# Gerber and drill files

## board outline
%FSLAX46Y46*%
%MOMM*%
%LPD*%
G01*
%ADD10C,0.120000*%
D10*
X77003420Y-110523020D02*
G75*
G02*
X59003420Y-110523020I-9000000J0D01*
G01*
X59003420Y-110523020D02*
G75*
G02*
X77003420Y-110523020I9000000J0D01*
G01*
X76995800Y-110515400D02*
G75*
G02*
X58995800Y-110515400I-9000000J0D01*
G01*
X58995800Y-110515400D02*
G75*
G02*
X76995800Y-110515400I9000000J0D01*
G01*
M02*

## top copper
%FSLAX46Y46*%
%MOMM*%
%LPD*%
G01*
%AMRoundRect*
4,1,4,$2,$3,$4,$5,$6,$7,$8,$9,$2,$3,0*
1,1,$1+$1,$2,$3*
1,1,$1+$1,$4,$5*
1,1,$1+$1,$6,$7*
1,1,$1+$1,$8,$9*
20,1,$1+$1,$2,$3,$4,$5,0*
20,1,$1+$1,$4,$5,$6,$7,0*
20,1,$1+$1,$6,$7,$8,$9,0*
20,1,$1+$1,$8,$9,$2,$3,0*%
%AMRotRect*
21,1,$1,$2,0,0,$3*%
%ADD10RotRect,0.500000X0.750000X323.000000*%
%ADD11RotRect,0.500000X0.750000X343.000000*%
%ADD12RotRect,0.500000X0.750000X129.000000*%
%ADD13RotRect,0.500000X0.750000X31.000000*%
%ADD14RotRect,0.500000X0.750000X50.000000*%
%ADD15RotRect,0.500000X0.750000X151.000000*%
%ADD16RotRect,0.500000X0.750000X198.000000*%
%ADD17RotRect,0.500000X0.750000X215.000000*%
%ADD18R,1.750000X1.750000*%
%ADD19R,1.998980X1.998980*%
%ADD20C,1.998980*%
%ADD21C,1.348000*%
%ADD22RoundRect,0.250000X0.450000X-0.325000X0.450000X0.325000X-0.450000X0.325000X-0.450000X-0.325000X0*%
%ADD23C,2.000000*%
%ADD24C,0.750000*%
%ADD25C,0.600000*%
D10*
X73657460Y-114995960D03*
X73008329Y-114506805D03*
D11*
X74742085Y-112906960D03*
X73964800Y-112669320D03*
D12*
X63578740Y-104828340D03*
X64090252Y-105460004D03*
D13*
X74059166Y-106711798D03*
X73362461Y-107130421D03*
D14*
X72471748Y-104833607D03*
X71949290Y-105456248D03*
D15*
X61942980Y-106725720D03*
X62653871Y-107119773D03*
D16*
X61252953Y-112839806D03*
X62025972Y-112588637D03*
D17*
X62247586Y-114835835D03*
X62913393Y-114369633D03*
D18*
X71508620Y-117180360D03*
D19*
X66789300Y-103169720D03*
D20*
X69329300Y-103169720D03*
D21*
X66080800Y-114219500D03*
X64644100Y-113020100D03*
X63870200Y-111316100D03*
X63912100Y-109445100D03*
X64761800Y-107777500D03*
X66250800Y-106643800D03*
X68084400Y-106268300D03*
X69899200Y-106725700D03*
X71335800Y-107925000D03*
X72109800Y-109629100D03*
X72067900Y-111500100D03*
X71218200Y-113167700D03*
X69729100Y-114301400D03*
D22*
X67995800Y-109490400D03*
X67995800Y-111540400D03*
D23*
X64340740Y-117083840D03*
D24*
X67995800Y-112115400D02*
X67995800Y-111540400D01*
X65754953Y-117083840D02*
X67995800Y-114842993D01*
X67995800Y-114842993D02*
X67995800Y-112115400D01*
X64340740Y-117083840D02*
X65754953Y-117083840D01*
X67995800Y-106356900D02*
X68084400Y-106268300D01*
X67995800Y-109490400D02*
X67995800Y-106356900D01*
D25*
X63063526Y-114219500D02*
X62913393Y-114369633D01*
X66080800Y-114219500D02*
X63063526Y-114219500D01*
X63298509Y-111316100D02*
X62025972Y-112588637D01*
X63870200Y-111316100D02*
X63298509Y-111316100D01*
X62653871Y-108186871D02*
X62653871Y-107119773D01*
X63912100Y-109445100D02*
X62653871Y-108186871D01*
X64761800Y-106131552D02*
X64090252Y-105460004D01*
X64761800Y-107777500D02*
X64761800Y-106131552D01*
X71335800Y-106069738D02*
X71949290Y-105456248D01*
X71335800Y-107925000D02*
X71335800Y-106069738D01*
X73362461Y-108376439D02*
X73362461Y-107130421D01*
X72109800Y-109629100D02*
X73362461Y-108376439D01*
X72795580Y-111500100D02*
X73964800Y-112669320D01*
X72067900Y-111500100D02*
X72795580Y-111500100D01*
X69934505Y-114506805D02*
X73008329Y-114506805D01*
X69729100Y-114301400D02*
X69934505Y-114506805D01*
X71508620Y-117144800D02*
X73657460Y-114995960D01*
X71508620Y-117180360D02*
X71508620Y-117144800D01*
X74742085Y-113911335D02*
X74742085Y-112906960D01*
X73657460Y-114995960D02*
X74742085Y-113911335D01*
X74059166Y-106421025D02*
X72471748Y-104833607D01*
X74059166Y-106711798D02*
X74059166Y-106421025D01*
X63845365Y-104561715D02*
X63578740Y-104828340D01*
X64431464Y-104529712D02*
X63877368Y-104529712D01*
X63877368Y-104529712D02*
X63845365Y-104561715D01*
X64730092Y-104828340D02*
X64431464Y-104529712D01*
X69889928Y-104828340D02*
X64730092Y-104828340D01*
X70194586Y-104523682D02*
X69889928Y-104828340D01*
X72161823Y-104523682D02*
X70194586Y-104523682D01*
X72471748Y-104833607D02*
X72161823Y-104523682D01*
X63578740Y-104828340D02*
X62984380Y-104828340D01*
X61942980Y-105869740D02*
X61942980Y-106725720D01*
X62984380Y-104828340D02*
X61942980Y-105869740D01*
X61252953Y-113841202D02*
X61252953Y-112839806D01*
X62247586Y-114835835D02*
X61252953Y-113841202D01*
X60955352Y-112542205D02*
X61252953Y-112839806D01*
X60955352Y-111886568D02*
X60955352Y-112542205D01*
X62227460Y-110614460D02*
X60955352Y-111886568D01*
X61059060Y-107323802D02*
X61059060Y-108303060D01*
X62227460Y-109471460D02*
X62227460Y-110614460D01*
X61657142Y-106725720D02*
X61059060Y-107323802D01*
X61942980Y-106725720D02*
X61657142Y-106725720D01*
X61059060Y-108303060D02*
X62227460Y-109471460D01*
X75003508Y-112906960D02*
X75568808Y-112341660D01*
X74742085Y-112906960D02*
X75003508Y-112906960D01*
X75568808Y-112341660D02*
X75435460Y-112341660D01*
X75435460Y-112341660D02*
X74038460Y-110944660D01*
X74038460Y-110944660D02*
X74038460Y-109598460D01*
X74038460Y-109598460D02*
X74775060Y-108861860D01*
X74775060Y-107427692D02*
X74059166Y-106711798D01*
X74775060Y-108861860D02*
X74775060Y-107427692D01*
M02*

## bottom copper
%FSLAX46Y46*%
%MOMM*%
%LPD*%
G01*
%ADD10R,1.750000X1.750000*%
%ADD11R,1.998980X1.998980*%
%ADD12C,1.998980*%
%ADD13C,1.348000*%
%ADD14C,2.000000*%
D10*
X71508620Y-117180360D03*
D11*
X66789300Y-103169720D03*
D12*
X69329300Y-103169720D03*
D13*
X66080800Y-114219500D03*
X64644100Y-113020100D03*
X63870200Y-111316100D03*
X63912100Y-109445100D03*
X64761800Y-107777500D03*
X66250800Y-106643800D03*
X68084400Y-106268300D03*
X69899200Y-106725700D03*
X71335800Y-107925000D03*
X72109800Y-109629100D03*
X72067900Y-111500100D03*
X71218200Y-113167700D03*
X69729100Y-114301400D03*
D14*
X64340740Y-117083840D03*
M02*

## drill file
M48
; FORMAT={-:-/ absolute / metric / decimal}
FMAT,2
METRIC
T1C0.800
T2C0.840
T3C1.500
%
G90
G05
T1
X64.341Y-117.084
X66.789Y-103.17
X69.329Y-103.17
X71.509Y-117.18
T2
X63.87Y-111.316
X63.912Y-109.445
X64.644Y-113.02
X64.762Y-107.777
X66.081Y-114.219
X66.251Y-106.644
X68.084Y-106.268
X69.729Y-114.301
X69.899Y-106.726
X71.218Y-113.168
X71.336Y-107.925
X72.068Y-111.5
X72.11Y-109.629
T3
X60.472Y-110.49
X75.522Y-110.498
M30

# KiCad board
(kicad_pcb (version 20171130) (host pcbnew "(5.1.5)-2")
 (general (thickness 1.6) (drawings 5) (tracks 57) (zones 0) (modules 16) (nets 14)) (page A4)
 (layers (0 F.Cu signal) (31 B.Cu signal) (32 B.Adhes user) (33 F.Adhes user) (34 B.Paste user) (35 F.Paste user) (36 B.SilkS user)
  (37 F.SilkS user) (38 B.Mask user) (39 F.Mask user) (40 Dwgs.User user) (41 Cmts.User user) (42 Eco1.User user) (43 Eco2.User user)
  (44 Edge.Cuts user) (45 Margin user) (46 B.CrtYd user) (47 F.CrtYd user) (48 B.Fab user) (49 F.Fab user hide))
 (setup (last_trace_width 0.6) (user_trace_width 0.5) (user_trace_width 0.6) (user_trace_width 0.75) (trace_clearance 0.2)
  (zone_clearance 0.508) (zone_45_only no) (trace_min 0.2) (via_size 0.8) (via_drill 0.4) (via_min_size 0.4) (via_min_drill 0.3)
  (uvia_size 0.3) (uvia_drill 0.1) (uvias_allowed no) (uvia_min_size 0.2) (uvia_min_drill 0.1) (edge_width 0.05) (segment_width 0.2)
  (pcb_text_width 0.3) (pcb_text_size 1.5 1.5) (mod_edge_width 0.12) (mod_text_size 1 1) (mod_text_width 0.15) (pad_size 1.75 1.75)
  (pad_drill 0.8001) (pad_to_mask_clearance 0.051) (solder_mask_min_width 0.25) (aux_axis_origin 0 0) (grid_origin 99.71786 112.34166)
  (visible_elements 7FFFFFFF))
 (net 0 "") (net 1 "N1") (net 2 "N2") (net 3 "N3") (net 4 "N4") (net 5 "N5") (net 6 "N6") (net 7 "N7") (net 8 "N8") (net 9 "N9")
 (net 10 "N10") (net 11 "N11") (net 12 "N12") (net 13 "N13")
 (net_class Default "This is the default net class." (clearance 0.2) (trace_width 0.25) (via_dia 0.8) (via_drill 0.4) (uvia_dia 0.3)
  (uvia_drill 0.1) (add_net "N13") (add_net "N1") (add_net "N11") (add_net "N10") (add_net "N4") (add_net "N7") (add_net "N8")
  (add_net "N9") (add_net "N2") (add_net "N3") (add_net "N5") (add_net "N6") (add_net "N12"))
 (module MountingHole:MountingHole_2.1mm (layer F.Cu) (at 60.47232 110.49)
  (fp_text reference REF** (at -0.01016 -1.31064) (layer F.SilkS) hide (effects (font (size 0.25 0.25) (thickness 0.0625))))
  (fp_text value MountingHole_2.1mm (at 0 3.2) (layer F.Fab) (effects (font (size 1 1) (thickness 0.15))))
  (pad "" np_thru_hole circle (at 0 0) (size 1.5 1.5) (drill 1.5) (layers *.Cu *.Mask)))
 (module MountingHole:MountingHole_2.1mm (layer F.Cu) (at 75.52182 110.49762)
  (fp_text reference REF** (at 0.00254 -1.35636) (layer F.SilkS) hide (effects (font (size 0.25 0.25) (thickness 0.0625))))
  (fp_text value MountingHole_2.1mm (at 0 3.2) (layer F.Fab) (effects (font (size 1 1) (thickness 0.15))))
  (pad "" np_thru_hole circle (at 0 0) (size 1.5 1.5) (drill 1.5) (layers *.Cu *.Mask)))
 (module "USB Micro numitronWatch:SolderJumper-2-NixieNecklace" (layer F.Cu) (at 73.530749 114.868672 323)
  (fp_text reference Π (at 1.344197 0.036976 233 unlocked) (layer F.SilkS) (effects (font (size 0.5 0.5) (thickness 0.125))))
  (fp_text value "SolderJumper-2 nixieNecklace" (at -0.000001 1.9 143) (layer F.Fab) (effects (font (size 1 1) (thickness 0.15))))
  (pad 2 smd rect (at 0.1778 0.0254 323) (size 0.5 0.75) (layers F.Cu F.Mask) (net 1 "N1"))
  (pad 1 smd rect (at -0.635 0.0254 323) (size 0.5 0.75) (layers F.Cu F.Mask) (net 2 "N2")))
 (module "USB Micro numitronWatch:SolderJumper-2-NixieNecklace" (layer F.Cu) (at 74.57948 112.830686 343)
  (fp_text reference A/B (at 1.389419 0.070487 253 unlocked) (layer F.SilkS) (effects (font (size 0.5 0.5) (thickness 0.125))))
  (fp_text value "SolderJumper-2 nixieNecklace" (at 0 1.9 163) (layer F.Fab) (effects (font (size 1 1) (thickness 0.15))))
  (pad 2 smd rect (at 0.1778 0.0254 343) (size 0.5 0.75) (layers F.Cu F.Mask) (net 1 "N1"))
  (pad 1 smd rect (at -0.635 0.0254 343) (size 0.5 0.75) (layers F.Cu F.Mask) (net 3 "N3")))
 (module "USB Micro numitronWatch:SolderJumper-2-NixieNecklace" (layer F.Cu) (at 63.670894 104.982501 129)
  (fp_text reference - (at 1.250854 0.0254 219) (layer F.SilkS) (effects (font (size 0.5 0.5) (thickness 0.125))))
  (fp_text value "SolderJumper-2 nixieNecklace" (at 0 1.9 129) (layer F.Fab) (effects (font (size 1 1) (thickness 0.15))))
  (pad 2 smd rect (at 0.1778 0.0254 129) (size 0.5 0.75) (layers F.Cu F.Mask) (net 1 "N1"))
  (pad 1 smd rect (at -0.635 0.0254 129) (size 0.5 0.75) (layers F.Cu F.Mask) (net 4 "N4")))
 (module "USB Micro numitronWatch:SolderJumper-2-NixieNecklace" (layer F.Cu) (at 73.89368 106.7816 31)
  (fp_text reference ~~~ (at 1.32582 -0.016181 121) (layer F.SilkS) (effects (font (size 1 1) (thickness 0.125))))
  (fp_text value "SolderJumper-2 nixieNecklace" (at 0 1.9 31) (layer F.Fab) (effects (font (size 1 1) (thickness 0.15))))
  (pad 2 smd rect (at 0.1778 0.0254 31) (size 0.5 0.75) (layers F.Cu F.Mask) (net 1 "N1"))
  (pad 1 smd rect (at -0.635 0.0254 31) (size 0.5 0.75) (layers F.Cu F.Mask) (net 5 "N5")))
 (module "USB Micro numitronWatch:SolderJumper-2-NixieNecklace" (layer F.Cu) (at 72.338003 104.953483 50)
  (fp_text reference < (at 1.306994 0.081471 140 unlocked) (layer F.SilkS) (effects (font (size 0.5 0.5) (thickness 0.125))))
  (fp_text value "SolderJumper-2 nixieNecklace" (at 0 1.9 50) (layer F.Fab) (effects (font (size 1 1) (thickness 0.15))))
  (pad 2 smd rect (at 0.1778 0.0254 50) (size 0.5 0.75) (layers F.Cu F.Mask) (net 1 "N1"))
  (pad 1 smd rect (at -0.635 0.0254 50) (size 0.5 0.75) (layers F.Cu F.Mask) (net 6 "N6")))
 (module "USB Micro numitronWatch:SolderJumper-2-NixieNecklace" (layer F.Cu) (at 62.086173 106.834134 151)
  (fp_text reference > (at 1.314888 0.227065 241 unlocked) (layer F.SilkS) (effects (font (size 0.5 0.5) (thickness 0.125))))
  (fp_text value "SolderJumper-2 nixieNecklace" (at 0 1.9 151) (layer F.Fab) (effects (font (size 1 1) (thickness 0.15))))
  (pad 2 smd rect (at 0.1778 0.0254 151) (size 0.5 0.75) (layers F.Cu F.Mask) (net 1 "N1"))
  (pad 1 smd rect (at -0.635 0.0254 151) (size 0.5 0.75) (layers F.Cu F.Mask) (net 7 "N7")))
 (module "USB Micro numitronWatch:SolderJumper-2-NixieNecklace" (layer F.Cu) (at 61.4299 112.80902 198)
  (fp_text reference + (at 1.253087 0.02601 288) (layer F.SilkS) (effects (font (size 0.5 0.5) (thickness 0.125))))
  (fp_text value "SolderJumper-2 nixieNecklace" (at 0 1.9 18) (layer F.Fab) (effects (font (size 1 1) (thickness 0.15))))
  (pad 2 smd rect (at 0.1778 0.0254 198) (size 0.5 0.75) (layers F.Cu F.Mask) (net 1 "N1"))
  (pad 1 smd rect (at -0.635 0.0254 198) (size 0.5 0.75) (layers F.Cu F.Mask) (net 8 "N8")))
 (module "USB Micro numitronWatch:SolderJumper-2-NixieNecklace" (layer F.Cu) (at 62.4078 114.75466 215)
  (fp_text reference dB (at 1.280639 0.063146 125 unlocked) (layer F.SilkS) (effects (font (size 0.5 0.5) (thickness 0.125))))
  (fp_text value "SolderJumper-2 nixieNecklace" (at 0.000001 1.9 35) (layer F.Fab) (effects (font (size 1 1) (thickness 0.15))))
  (pad 2 smd rect (at 0.1778 0.0254 215) (size 0.5 0.75) (layers F.Cu F.Mask) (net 1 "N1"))
  (pad 1 smd rect (at -0.635 0.0254 215) (size 0.5 0.75) (layers F.Cu F.Mask) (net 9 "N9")))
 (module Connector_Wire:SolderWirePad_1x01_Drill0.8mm (layer F.Cu) (at 71.50862 117.18036)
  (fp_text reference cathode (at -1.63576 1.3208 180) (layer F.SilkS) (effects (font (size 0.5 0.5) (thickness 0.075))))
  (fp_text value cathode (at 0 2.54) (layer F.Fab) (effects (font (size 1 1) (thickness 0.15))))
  (pad 1 thru_hole rect (at 0 0) (size 1.75 1.75) (drill 0.8001) (layers *.Cu *.Mask) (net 1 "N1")))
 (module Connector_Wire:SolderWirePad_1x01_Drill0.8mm (layer F.Cu) (at 66.7893 103.16972)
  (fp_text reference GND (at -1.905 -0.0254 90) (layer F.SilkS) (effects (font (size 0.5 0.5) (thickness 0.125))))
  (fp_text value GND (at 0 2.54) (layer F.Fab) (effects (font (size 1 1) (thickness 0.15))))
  (pad 1 thru_hole rect (at 0 0) (size 1.99898 1.99898) (drill 0.8001) (layers *.Cu *.Mask) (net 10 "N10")))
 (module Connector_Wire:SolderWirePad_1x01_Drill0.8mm (layer F.Cu) (at 69.3293 103.16972)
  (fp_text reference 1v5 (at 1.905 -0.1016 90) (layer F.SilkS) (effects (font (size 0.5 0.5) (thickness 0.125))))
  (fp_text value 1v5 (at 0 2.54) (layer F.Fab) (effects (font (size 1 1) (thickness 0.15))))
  (pad 1 thru_hole circle (at 0 0) (size 1.99898 1.99898) (drill 0.8001) (layers *.Cu *.Mask) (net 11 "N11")))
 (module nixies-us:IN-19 (layer F.Cu) (at 67.9958 110.5154)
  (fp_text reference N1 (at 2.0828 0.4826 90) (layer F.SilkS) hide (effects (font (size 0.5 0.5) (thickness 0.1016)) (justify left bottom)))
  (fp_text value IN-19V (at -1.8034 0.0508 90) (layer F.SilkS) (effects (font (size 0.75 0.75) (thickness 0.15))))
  (pad 14 thru_hole circle (at -1.915 3.7041 333) (size 1.348 1.348) (drill 0.84) (layers *.Cu *.Mask) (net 9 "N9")
   (solder_mask_margin 0.1016))
  (pad 13 thru_hole circle (at -3.3517 2.5047 333) (size 1.348 1.348) (drill 0.84) (layers *.Cu *.Mask) (solder_mask_margin 0.1016))
  (pad 12 thru_hole circle (at -4.1256 0.8007 333) (size 1.348 1.348) (drill 0.84) (layers *.Cu *.Mask) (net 8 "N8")
   (solder_mask_margin 0.1016))
  (pad 11 thru_hole circle (at -4.0837 -1.0703 333) (size 1.348 1.348) (drill 0.84) (layers *.Cu *.Mask) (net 7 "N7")
   (solder_mask_margin 0.1016))
  (pad 10 thru_hole circle (at -3.234 -2.7379 333) (size 1.348 1.348) (drill 0.84) (layers *.Cu *.Mask) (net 4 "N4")
   (solder_mask_margin 0.1016))
  (pad 9 thru_hole circle (at -1.745 -3.8716 333) (size 1.348 1.348) (drill 0.84) (layers *.Cu *.Mask) (solder_mask_margin 0.1016))
  (pad 8 thru_hole circle (at 0.0886 -4.2471 333) (size 1.348 1.348) (drill 0.84) (layers *.Cu *.Mask) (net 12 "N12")
   (solder_mask_margin 0.1016))
  (pad 7 thru_hole circle (at 1.9034 -3.7897 333) (size 1.348 1.348) (drill 0.84) (layers *.Cu *.Mask) (solder_mask_margin 0.1016))
  (pad 6 thru_hole circle (at 3.34 -2.5904 333) (size 1.348 1.348) (drill 0.84) (layers *.Cu *.Mask) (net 6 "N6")
   (solder_mask_margin 0.1016))
  (pad 5 thru_hole circle (at 4.114 -0.8863 333) (size 1.348 1.348) (drill 0.84) (layers *.Cu *.Mask) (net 5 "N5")
   (solder_mask_margin 0.1016))
  (pad 4 thru_hole circle (at 4.0721 0.9847 333) (size 1.348 1.348) (drill 0.84) (layers *.Cu *.Mask) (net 3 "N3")
   (solder_mask_margin 0.1016))
  (pad 3 thru_hole circle (at 3.2224 2.6523 333) (size 1.348 1.348) (drill 0.84) (layers *.Cu *.Mask) (solder_mask_margin 0.1016))
  (pad 2 thru_hole circle (at 1.7333 3.786 333) (size 1.348 1.348) (drill 0.84) (layers *.Cu *.Mask) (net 2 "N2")
   (solder_mask_margin 0.1016)))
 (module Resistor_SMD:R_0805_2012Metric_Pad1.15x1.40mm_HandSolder (layer F.Cu) (at 67.9958 110.5154 90)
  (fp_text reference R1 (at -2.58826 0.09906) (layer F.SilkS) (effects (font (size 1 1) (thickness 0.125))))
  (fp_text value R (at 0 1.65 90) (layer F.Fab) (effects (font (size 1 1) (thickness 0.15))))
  (pad 2 smd roundrect (at 1.025 0 90) (size 1.15 1.4) (layers F.Cu F.Paste F.Mask) (roundrect_rratio 0.217391) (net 12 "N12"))
  (pad 1 smd roundrect (at -1.025 0 90) (size 1.15 1.4) (layers F.Cu F.Paste F.Mask) (roundrect_rratio 0.217391) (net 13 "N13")))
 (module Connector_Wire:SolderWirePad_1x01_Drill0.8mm (layer F.Cu) (at 64.34074 117.08384)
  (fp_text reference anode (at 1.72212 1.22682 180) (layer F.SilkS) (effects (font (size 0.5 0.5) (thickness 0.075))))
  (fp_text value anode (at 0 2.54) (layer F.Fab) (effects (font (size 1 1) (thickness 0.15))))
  (pad 1 thru_hole circle (at 0 0) (size 2 2) (drill 0.8001) (layers *.Cu *.Mask) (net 13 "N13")))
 (gr_circle (center 68.00342 110.52302) (end 77.00342 110.52302) (layer Edge.Cuts) (width 0.12))
 (gr_circle (center 67.9958 110.5154) (end 76.9958 110.5154) (layer Edge.Cuts) (width 0.12))
 (segment (start 67.9958 112.1154) (end 67.9958 111.5404) (width 0.75) (layer F.Cu) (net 13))
 (segment (start 65.754953 117.08384) (end 67.9958 114.842993) (width 0.75) (layer F.Cu) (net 13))
 (segment (start 67.9958 114.842993) (end 67.9958 112.1154) (width 0.75) (layer F.Cu) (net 13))
 (segment (start 64.34074 117.08384) (end 65.754953 117.08384) (width 0.75) (layer F.Cu) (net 13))
 (segment (start 67.9958 106.3569) (end 68.0844 106.2683) (width 0.75) (layer F.Cu) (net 12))
 (segment (start 67.9958 109.4904) (end 67.9958 106.3569) (width 0.75) (layer F.Cu) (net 12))
 (segment (start 63.063526 114.2195) (end 62.913393 114.369633) (width 0.6) (layer F.Cu) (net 9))
 (segment (start 66.0808 114.2195) (end 63.063526 114.2195) (width 0.6) (layer F.Cu) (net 9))
 (segment (start 63.298509 111.3161) (end 62.025972 112.588637) (width 0.6) (layer F.Cu) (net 8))
 (segment (start 63.8702 111.3161) (end 63.298509 111.3161) (width 0.6) (layer F.Cu) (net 8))
 (segment (start 62.653871 108.186871) (end 62.653871 107.119773) (width 0.6) (layer F.Cu) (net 7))
 (segment (start 63.9121 109.4451) (end 62.653871 108.186871) (width 0.6) (layer F.Cu) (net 7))
 (segment (start 64.7618 106.131552) (end 64.090252 105.460004) (width 0.6) (layer F.Cu) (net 4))
 (segment (start 64.7618 107.7775) (end 64.7618 106.131552) (width 0.6) (layer F.Cu) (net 4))
 (segment (start 71.3358 106.069738) (end 71.94929 105.456248) (width 0.6) (layer F.Cu) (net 6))
 (segment (start 71.3358 107.925) (end 71.3358 106.069738) (width 0.6) (layer F.Cu) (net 6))
 (segment (start 73.362461 108.376439) (end 73.362461 107.130421) (width 0.6) (layer F.Cu) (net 5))
 (segment (start 72.1098 109.6291) (end 73.362461 108.376439) (width 0.6) (layer F.Cu) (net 5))
 (segment (start 72.79558 111.5001) (end 73.9648 112.66932) (width 0.6) (layer F.Cu) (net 3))
 (segment (start 72.0679 111.5001) (end 72.79558 111.5001) (width 0.6) (layer F.Cu) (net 3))
 (segment (start 69.934505 114.506805) (end 73.008329 114.506805) (width 0.6) (layer F.Cu) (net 2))
 (segment (start 69.7291 114.3014) (end 69.934505 114.506805) (width 0.6) (layer F.Cu) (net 2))
 (segment (start 71.50862 117.1448) (end 73.65746 114.99596) (width 0.6) (layer F.Cu) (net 1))
 (segment (start 71.50862 117.18036) (end 71.50862 117.1448) (width 0.6) (layer F.Cu) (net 1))
 (segment (start 74.742085 113.911335) (end 74.742085 112.90696) (width 0.6) (layer F.Cu) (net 1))
 (segment (start 73.65746 114.99596) (end 74.742085 113.911335) (width 0.6) (layer F.Cu) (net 1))
 (segment (start 74.059166 106.421025) (end 72.471748 104.833607) (width 0.6) (layer F.Cu) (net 1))
 (segment (start 74.059166 106.711798) (end 74.059166 106.421025) (width 0.6) (layer F.Cu) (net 1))
 (segment (start 63.845365 104.561715) (end 63.57874 104.82834) (width 0.6) (layer F.Cu) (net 1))
 (segment (start 64.431464 104.529712) (end 63.877368 104.529712) (width 0.6) (layer F.Cu) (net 1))
 (segment (start 63.877368 104.529712) (end 63.845365 104.561715) (width 0.6) (layer F.Cu) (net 1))
 (segment (start 64.730092 104.82834) (end 64.431464 104.529712) (width 0.6) (layer F.Cu) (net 1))
 (segment (start 69.889928 104.82834) (end 64.730092 104.82834) (width 0.6) (layer F.Cu) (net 1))
 (segment (start 70.194586 104.523682) (end 69.889928 104.82834) (width 0.6) (layer F.Cu) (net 1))
 (segment (start 72.161823 104.523682) (end 70.194586 104.523682) (width 0.6) (layer F.Cu) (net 1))
 (segment (start 72.471748 104.833607) (end 72.161823 104.523682) (width 0.6) (layer F.Cu) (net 1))
 (segment (start 63.57874 104.82834) (end 62.98438 104.82834) (width 0.6) (layer F.Cu) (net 1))
 (segment (start 61.94298 105.86974) (end 61.94298 106.72572) (width 0.6) (layer F.Cu) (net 1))
 (segment (start 62.98438 104.82834) (end 61.94298 105.86974) (width 0.6) (layer F.Cu) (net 1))
 (segment (start 61.252953 113.841202) (end 61.252953 112.839806) (width 0.6) (layer F.Cu) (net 1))
 (segment (start 62.247586 114.835835) (end 61.252953 113.841202) (width 0.6) (layer F.Cu) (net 1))
 (segment (start 60.955352 112.542205) (end 61.252953 112.839806) (width 0.6) (layer F.Cu) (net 1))
 (segment (start 60.955352 111.886568) (end 60.955352 112.542205) (width 0.6) (layer F.Cu) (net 1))
 (segment (start 62.22746 110.61446) (end 60.955352 111.886568) (width 0.6) (layer F.Cu) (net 1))
 (segment (start 61.05906 107.323802) (end 61.05906 108.30306) (width 0.6) (layer F.Cu) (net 1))
 (segment (start 62.22746 109.47146) (end 62.22746 110.61446) (width 0.6) (layer F.Cu) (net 1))
 (segment (start 61.657142 106.72572) (end 61.05906 107.323802) (width 0.6) (layer F.Cu) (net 1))
 (segment (start 61.94298 106.72572) (end 61.657142 106.72572) (width 0.6) (layer F.Cu) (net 1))
 (segment (start 61.05906 108.30306) (end 62.22746 109.47146) (width 0.6) (layer F.Cu) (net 1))
 (segment (start 75.003508 112.90696) (end 75.568808 112.34166) (width 0.6) (layer F.Cu) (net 1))
 (segment (start 74.742085 112.90696) (end 75.003508 112.90696) (width 0.6) (layer F.Cu) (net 1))
 (segment (start 75.568808 112.34166) (end 75.43546 112.34166) (width 0.6) (layer F.Cu) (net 1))
 (segment (start 75.43546 112.34166) (end 74.03846 110.94466) (width 0.6) (layer F.Cu) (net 1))
 (segment (start 74.03846 110.94466) (end 74.03846 109.59846) (width 0.6) (layer F.Cu) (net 1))
 (segment (start 74.03846 109.59846) (end 74.77506 108.86186) (width 0.6) (layer F.Cu) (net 1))
 (segment (start 74.77506 107.427692) (end 74.059166 106.711798) (width 0.6) (layer F.Cu) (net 1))
 (segment (start 74.77506 108.86186) (end 74.77506 107.427692) (width 0.6) (layer F.Cu) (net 1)))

